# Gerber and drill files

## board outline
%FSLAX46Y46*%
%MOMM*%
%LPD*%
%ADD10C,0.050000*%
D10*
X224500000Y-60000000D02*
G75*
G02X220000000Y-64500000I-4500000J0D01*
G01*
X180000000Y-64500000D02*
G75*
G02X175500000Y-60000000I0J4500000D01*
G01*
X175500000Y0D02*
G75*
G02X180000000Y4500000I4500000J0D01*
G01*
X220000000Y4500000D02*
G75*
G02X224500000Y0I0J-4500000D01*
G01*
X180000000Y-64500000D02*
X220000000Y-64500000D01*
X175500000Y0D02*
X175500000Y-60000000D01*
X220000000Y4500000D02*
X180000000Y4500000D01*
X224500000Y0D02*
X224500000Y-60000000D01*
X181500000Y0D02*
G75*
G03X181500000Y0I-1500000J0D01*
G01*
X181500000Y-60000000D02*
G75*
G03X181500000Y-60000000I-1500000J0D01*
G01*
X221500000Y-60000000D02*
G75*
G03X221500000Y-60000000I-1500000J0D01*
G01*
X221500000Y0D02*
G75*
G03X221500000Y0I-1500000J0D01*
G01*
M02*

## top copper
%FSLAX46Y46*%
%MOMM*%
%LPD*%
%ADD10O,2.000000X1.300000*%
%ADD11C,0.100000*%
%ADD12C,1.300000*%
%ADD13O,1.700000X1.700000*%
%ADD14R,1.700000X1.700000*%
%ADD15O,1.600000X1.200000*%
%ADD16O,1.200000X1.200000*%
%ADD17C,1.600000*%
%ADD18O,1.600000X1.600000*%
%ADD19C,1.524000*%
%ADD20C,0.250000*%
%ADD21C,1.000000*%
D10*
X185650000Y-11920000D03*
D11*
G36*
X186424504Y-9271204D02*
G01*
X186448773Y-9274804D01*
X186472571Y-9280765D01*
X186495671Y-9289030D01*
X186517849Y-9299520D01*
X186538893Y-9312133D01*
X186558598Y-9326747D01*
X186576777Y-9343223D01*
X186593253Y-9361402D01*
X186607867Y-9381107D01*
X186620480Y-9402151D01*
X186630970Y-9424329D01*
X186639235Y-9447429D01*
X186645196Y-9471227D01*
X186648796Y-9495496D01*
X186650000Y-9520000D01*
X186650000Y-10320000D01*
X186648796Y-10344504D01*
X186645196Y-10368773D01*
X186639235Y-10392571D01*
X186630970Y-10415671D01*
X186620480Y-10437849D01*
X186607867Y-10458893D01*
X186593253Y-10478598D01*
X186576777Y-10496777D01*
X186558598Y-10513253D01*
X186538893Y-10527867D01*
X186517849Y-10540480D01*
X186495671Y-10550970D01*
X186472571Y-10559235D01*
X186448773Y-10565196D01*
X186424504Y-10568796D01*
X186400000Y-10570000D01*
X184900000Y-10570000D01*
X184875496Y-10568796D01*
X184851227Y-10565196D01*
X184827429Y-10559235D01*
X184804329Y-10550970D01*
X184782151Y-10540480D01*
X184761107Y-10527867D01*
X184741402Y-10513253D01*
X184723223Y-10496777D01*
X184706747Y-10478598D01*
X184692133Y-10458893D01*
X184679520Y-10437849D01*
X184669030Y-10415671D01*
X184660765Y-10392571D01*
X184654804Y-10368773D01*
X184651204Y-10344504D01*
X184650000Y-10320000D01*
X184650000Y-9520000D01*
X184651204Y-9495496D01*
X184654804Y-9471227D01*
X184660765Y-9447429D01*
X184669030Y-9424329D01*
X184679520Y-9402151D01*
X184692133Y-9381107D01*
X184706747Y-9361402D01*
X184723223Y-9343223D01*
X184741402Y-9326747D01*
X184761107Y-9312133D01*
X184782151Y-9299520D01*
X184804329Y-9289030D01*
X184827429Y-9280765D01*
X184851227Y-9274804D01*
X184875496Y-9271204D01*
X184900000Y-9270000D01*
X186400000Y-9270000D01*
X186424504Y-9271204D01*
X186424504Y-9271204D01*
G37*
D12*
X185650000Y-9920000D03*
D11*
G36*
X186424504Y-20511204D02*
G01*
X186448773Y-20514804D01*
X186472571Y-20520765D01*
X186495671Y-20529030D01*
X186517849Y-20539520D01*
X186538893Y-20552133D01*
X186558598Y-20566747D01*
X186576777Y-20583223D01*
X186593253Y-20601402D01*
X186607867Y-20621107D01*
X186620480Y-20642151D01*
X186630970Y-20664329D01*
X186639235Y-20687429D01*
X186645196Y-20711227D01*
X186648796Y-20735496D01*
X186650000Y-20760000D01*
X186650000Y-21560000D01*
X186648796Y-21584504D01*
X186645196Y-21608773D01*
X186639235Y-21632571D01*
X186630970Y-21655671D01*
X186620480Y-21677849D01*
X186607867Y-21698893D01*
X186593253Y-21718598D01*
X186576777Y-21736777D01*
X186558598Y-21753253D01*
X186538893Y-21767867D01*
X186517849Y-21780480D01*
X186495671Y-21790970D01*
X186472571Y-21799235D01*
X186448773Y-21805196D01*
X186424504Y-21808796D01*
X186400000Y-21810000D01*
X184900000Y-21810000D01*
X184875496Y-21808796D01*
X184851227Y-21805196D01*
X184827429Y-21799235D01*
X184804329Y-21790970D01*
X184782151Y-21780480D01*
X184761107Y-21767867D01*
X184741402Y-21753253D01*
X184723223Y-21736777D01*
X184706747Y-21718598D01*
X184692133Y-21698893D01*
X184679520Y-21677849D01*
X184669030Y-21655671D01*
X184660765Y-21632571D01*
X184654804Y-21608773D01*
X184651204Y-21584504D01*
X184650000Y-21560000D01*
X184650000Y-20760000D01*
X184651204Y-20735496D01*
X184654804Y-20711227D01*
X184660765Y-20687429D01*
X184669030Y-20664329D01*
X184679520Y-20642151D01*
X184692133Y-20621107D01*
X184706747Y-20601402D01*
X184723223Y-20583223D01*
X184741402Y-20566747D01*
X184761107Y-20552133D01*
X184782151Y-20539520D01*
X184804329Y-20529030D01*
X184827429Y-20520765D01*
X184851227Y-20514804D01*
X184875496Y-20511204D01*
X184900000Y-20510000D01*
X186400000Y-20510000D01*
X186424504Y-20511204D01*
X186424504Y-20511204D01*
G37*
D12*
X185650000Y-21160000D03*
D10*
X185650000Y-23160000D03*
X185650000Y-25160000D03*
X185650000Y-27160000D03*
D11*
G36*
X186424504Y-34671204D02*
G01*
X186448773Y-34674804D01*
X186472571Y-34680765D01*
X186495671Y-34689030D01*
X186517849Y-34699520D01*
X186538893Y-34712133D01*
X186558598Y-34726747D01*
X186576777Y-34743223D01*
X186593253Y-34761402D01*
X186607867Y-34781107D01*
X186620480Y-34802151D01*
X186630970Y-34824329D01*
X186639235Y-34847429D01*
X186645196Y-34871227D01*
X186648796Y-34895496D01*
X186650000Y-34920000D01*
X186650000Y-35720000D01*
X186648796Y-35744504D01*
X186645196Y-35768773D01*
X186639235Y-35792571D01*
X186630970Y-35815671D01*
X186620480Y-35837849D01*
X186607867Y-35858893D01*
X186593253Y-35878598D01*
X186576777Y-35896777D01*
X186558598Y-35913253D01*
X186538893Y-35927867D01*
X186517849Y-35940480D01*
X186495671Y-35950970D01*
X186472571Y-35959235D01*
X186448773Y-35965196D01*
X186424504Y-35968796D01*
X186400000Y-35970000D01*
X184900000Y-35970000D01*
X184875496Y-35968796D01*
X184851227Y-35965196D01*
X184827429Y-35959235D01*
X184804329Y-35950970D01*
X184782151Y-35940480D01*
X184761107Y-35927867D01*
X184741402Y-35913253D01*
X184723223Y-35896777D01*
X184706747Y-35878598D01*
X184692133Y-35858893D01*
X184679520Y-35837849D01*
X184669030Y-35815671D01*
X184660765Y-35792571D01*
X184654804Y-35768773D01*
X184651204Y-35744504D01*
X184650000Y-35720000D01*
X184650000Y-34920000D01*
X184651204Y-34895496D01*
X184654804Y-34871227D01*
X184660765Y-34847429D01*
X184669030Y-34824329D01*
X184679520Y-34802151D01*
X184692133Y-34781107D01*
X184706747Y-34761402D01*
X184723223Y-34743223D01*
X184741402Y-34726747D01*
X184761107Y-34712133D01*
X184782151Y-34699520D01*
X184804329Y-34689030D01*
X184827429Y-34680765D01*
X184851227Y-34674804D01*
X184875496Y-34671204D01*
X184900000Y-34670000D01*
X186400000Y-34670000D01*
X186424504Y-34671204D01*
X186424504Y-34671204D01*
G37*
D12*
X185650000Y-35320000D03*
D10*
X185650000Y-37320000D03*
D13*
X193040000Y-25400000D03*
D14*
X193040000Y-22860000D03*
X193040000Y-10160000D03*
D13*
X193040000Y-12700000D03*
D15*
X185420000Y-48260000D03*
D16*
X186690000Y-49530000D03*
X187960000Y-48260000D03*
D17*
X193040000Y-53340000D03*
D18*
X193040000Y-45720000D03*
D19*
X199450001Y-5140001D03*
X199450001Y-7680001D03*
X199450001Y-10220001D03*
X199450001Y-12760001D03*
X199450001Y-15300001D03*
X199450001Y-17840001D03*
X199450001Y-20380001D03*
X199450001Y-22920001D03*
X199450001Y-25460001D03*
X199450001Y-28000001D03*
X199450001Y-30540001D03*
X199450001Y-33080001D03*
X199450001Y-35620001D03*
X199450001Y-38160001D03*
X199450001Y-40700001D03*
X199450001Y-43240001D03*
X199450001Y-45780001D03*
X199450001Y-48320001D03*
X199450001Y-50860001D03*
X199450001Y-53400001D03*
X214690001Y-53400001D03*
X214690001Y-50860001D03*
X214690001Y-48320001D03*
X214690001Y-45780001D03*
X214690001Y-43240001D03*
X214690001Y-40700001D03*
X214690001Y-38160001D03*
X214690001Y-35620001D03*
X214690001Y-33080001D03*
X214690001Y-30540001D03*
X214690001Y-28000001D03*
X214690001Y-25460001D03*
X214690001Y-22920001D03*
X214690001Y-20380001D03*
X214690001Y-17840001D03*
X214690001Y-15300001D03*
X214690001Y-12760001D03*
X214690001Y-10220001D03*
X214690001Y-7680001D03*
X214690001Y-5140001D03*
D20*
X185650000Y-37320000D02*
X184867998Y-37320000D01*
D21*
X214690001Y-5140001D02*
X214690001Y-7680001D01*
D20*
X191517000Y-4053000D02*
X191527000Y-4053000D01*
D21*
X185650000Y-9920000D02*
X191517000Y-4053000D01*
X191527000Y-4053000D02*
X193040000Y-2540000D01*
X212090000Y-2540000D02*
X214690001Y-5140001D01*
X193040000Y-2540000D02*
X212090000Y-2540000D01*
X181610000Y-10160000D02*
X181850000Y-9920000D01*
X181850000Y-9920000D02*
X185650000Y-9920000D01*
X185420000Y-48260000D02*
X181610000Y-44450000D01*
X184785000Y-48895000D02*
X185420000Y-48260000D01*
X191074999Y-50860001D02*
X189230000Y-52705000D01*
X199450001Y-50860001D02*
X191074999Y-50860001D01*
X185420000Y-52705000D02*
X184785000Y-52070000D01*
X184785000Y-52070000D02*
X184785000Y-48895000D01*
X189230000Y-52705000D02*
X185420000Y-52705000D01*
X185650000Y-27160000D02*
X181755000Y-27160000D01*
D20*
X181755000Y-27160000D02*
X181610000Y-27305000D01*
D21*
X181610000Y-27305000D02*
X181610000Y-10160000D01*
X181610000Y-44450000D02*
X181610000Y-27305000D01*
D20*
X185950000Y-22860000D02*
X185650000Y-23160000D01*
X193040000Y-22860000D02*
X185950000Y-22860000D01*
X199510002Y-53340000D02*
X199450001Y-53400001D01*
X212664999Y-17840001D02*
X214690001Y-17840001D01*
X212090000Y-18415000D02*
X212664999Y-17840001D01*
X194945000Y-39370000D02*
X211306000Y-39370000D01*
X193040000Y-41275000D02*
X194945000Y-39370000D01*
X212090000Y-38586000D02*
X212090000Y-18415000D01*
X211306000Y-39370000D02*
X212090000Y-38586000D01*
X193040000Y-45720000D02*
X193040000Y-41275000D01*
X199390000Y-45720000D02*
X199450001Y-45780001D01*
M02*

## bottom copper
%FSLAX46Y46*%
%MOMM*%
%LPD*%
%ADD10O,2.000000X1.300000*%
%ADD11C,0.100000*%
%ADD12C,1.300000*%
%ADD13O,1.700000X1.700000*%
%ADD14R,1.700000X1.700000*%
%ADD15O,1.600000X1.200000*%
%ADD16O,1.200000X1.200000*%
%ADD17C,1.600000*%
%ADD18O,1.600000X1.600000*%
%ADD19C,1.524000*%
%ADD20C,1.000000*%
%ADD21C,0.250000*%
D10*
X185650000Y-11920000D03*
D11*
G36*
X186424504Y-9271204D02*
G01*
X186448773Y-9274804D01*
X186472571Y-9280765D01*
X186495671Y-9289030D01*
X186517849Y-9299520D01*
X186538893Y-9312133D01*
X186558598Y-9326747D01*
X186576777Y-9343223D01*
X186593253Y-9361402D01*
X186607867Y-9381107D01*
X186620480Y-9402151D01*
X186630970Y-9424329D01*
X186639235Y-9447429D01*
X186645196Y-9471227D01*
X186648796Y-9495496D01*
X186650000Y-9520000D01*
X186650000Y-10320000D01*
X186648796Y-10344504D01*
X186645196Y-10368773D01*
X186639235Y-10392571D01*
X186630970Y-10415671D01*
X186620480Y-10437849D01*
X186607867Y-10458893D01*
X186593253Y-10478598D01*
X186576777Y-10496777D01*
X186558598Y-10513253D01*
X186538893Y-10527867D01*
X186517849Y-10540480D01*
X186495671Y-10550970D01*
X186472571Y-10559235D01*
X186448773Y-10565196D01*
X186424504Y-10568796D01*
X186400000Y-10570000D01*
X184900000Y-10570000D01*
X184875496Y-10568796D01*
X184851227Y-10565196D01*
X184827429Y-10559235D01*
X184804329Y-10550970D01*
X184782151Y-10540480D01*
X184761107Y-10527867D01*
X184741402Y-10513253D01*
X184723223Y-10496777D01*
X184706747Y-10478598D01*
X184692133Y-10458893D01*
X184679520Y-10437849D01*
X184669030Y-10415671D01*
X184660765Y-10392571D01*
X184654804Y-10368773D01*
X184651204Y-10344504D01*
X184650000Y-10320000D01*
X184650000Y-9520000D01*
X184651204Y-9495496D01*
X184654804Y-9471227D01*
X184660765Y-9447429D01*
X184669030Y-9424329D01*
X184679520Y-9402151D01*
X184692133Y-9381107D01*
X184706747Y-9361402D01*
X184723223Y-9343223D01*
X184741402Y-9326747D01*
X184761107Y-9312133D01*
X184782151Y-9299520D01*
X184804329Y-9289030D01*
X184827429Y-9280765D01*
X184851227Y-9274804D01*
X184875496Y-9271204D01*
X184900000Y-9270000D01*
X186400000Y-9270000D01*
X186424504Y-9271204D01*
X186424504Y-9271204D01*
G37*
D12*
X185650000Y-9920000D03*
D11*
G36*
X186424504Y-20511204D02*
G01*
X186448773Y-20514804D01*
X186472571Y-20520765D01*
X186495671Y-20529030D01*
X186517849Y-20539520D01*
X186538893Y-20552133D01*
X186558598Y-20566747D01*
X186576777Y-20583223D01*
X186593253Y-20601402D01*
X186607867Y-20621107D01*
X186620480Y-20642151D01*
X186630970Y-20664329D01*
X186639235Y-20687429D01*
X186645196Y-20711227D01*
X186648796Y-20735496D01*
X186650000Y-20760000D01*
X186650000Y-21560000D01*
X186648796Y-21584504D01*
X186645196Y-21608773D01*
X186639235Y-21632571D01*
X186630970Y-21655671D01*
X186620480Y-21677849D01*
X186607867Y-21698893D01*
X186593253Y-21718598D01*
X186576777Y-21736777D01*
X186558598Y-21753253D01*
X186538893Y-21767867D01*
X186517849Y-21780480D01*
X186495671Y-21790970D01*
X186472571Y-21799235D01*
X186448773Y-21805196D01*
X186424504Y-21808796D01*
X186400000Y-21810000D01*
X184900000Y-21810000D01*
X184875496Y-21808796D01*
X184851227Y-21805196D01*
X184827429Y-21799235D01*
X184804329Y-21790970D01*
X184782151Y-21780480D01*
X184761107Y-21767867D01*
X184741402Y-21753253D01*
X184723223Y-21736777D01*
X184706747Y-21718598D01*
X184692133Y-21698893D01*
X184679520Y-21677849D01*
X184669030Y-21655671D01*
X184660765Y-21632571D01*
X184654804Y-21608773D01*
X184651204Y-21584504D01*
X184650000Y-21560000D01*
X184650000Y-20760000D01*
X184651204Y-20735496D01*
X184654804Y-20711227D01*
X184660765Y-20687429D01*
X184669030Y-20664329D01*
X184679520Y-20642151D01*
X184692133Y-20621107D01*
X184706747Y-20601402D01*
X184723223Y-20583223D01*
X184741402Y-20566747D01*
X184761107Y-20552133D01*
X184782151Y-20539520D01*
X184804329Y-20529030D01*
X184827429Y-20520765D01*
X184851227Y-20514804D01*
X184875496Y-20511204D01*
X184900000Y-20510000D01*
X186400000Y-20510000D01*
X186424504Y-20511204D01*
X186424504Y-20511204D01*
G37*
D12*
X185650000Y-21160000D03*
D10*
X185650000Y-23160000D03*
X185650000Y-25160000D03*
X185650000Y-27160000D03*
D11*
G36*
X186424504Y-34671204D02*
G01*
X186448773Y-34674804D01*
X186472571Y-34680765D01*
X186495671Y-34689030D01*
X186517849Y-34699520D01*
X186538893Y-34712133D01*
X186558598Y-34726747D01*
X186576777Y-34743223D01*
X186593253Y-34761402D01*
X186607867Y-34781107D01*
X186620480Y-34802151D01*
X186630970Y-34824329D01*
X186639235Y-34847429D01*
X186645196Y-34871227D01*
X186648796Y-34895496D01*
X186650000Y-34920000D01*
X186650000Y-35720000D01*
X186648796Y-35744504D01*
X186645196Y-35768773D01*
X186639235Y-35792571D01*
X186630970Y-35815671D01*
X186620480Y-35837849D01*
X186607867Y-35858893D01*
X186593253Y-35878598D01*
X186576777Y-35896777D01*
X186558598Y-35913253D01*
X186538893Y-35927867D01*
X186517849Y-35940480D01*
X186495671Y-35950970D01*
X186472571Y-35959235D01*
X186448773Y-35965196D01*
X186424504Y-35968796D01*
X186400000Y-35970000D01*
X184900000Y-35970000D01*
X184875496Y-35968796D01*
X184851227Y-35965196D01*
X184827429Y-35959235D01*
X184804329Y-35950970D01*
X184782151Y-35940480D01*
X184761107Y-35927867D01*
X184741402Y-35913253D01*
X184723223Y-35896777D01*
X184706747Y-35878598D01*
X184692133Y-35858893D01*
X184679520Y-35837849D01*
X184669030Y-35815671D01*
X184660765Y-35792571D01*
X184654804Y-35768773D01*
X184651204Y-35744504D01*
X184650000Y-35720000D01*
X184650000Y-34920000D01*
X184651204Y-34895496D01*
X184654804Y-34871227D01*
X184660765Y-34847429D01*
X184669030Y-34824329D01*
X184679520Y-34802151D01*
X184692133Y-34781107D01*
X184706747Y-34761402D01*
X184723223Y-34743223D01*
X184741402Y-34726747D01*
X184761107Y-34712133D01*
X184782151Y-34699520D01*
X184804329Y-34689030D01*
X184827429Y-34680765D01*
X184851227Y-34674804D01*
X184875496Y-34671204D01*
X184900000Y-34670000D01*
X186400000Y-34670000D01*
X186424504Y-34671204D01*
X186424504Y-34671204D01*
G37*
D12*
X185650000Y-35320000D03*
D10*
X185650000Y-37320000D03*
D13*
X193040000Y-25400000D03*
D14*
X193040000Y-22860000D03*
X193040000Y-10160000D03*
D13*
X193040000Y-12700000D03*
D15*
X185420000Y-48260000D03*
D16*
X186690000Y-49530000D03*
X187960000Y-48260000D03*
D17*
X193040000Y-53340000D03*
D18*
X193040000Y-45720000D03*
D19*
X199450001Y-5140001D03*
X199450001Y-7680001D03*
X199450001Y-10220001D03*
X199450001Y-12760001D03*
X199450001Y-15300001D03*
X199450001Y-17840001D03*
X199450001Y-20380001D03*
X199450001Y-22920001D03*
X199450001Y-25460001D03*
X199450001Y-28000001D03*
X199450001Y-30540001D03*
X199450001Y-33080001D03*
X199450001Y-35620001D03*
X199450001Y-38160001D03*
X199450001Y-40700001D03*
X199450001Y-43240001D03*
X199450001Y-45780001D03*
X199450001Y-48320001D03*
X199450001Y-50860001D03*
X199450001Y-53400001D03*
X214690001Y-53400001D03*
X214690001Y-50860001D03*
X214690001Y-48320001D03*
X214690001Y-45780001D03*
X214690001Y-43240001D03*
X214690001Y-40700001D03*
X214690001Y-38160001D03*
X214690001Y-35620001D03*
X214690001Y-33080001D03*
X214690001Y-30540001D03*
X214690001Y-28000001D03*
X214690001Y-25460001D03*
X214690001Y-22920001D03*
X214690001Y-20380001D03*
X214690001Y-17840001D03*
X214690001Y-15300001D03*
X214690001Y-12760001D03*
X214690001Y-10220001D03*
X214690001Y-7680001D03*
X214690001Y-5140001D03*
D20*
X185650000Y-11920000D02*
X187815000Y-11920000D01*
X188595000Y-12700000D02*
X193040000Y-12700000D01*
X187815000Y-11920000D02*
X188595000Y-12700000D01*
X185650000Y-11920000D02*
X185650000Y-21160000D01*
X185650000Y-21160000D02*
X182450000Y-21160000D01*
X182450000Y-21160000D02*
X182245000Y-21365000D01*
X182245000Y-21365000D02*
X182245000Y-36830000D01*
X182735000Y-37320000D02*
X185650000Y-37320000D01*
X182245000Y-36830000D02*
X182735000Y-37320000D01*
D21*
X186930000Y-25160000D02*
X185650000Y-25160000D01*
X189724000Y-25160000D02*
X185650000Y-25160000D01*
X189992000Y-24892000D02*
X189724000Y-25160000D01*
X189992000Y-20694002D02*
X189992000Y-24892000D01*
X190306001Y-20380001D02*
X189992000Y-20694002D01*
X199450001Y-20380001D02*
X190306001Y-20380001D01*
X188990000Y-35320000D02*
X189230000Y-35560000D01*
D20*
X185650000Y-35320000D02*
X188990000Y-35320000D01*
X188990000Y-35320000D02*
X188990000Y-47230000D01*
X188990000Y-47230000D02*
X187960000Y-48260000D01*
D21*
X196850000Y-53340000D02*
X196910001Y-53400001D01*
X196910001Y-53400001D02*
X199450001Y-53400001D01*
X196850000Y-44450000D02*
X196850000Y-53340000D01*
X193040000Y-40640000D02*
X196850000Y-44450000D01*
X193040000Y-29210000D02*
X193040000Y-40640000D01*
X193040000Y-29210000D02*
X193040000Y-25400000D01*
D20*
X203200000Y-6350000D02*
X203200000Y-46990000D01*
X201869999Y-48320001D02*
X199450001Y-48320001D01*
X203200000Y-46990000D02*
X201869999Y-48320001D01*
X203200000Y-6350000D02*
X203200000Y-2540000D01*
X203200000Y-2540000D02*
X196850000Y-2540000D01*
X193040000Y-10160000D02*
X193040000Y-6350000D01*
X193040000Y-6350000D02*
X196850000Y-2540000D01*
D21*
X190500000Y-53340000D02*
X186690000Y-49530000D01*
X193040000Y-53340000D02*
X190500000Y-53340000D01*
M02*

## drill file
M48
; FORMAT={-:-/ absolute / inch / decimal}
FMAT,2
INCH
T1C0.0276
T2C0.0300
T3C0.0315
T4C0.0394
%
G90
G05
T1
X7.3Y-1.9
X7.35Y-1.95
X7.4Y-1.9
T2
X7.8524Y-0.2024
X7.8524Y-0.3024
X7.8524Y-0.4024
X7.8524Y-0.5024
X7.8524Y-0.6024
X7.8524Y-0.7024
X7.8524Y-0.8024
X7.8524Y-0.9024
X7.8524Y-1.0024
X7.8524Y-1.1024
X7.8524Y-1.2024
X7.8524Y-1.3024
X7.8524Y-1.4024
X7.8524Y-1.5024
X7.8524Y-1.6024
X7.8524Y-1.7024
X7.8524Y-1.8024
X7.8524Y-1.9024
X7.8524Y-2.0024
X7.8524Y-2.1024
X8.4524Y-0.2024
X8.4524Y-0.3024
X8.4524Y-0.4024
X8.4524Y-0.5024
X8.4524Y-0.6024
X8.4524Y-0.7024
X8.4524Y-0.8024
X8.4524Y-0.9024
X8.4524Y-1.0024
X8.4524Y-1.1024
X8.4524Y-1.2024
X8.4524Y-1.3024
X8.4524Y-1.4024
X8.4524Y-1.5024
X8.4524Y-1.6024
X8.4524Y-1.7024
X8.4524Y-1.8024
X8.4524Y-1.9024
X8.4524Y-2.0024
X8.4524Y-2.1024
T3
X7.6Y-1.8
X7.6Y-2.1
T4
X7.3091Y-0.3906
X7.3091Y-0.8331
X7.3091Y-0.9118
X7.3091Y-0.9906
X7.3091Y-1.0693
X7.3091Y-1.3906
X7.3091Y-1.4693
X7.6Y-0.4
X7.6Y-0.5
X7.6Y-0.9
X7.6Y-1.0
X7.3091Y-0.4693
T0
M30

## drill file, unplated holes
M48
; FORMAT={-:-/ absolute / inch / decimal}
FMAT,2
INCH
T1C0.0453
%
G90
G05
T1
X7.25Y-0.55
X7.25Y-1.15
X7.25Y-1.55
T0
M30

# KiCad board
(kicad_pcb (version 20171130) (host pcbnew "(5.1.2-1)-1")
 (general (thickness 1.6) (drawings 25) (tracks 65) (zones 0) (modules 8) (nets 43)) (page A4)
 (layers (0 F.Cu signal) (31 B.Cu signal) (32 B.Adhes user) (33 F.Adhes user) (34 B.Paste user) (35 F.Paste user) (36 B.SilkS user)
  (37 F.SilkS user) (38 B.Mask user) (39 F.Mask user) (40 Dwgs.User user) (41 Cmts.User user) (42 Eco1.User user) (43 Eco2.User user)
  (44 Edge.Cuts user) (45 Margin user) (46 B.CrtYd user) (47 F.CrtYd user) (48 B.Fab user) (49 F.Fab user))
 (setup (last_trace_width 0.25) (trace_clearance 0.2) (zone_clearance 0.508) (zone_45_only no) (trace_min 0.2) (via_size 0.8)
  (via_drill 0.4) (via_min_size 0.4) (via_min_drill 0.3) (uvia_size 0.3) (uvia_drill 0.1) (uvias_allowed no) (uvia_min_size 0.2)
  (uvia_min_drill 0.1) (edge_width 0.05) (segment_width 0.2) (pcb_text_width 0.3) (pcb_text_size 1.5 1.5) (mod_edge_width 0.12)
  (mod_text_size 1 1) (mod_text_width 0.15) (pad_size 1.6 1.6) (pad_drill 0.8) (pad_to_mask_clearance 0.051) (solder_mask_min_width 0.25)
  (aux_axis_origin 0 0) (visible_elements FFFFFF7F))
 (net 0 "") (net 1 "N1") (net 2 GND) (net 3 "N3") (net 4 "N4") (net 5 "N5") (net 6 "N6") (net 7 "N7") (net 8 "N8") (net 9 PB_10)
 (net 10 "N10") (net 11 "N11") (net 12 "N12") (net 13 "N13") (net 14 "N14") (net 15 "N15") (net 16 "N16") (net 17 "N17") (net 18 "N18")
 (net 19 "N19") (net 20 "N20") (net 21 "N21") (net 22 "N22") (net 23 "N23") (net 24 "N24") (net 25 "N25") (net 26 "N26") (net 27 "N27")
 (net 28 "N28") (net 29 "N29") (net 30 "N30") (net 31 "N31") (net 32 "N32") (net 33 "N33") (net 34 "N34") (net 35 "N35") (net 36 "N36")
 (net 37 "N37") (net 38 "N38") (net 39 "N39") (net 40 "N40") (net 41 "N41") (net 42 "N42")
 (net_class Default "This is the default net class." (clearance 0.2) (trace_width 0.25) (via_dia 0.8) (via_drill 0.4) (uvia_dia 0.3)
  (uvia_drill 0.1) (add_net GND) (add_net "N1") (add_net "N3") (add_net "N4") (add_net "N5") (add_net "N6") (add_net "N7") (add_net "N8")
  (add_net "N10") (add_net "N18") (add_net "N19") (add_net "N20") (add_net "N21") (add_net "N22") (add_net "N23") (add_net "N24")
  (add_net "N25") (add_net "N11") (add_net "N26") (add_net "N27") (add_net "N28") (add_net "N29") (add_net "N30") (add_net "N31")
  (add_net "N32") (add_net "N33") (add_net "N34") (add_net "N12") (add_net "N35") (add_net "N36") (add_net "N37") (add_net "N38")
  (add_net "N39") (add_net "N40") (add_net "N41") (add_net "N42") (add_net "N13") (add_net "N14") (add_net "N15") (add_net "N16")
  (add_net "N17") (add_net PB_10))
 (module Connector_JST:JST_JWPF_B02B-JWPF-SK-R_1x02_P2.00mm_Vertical (layer F.Cu) (at 185.65 9.92)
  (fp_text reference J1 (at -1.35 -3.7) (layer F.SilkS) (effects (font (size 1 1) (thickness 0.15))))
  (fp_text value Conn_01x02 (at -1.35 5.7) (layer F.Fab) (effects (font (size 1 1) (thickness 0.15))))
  (pad "" np_thru_hole circle (at -1.5 4.05) (size 1.15 1.15) (drill 1.15) (layers *.Cu *.Mask))
  (pad 2 thru_hole oval (at 0 2) (size 2 1.3) (drill 1) (layers *.Cu *.Mask) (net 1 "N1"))
  (pad 1 thru_hole roundrect (at 0 0) (size 2 1.3) (drill 1) (layers *.Cu *.Mask) (roundrect_rratio 0.192308) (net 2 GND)))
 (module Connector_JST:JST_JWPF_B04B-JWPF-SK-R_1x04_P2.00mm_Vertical (layer F.Cu) (at 185.65 21.16)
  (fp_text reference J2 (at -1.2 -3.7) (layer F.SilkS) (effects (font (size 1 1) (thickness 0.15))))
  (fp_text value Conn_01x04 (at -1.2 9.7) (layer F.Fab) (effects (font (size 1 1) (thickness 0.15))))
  (pad 1 thru_hole roundrect (at 0 0) (size 2 1.3) (drill 1) (layers *.Cu *.Mask) (roundrect_rratio 0.192308) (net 1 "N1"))
  (pad 2 thru_hole oval (at 0 2) (size 2 1.3) (drill 1) (layers *.Cu *.Mask) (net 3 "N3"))
  (pad 3 thru_hole oval (at 0 4) (size 2 1.3) (drill 1) (layers *.Cu *.Mask) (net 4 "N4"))
  (pad 4 thru_hole oval (at 0 6) (size 2 1.3) (drill 1) (layers *.Cu *.Mask) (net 2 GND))
  (pad "" np_thru_hole circle (at -1.5 8.05) (size 1.15 1.15) (drill 1.15) (layers *.Cu *.Mask)))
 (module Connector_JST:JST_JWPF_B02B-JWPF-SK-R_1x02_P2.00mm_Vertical (layer F.Cu) (at 185.65 35.32)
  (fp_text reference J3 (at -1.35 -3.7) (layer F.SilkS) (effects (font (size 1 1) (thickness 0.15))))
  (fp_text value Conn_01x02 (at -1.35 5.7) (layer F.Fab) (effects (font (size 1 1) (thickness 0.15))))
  (pad 1 thru_hole roundrect (at 0 0) (size 2 1.3) (drill 1) (layers *.Cu *.Mask) (roundrect_rratio 0.192308) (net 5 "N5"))
  (pad 2 thru_hole oval (at 0 2) (size 2 1.3) (drill 1) (layers *.Cu *.Mask) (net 1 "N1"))
  (pad "" np_thru_hole circle (at -1.5 4.05) (size 1.15 1.15) (drill 1.15) (layers *.Cu *.Mask)))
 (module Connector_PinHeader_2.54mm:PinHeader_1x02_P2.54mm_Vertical (layer F.Cu) (at 193.04 22.86)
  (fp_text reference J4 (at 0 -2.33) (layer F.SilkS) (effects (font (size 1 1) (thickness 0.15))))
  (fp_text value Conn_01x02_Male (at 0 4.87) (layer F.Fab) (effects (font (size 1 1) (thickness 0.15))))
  (pad 2 thru_hole oval (at 0 2.54) (size 1.7 1.7) (drill 1) (layers *.Cu *.Mask) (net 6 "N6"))
  (pad 1 thru_hole rect (at 0 0) (size 1.7 1.7) (drill 1) (layers *.Cu *.Mask) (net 3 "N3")))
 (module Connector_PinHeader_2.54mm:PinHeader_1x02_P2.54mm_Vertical (layer F.Cu) (at 193.04 10.16)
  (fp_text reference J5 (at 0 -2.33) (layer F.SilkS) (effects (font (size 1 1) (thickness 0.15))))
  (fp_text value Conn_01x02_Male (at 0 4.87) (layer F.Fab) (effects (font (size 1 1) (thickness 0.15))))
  (pad 1 thru_hole rect (at 0 0) (size 1.7 1.7) (drill 1) (layers *.Cu *.Mask) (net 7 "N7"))
  (pad 2 thru_hole oval (at 0 2.54) (size 1.7 1.7) (drill 1) (layers *.Cu *.Mask) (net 1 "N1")))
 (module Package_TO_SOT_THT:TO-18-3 (layer F.Cu) (at 185.42 48.26)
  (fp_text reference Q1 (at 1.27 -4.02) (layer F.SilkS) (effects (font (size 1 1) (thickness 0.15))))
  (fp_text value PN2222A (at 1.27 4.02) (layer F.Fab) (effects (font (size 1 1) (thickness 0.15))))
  (pad 1 thru_hole oval (at 0 0) (size 1.6 1.2) (drill 0.7) (layers *.Cu *.Mask) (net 2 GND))
  (pad 2 thru_hole oval (at 1.27 1.27) (size 1.2 1.2) (drill 0.7) (layers *.Cu *.Mask) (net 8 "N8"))
  (pad 3 thru_hole oval (at 2.54 0) (size 1.2 1.2) (drill 0.7) (layers *.Cu *.Mask) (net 5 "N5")))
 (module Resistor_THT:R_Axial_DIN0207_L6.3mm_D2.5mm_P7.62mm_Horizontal (layer F.Cu) (at 193.04 53.34 90)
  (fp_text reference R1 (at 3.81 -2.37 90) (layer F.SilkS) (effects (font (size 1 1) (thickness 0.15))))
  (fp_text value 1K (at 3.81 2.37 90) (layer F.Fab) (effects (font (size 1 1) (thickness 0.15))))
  (pad 1 thru_hole circle (at 0 0 90) (size 1.6 1.6) (drill 0.8) (layers *.Cu *.Mask) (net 8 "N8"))
  (pad 2 thru_hole oval (at 7.62 0 90) (size 1.6 1.6) (drill 0.8) (layers *.Cu *.Mask) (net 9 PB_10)))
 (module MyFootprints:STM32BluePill (layer F.Cu) (at 199.450001 5.140001)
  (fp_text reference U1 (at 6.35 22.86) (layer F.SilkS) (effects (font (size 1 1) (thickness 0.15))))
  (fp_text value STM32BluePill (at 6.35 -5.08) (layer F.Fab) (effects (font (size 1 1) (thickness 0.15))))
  (pad 1 thru_hole circle (at 0 0) (size 1.524 1.524) (drill 0.762) (layers *.Cu *.Mask) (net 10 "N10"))
  (pad 2 thru_hole circle (at 0 2.54) (size 1.524 1.524) (drill 0.762) (layers *.Cu *.Mask) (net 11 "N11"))
  (pad 3 thru_hole circle (at 0 5.08) (size 1.524 1.524) (drill 0.762) (layers *.Cu *.Mask) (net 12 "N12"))
  (pad 4 thru_hole circle (at 0 7.62) (size 1.524 1.524) (drill 0.762) (layers *.Cu *.Mask) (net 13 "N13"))
  (pad 5 thru_hole circle (at 0 10.16) (size 1.524 1.524) (drill 0.762) (layers *.Cu *.Mask) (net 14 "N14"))
  (pad 6 thru_hole circle (at 0 12.7) (size 1.524 1.524) (drill 0.762) (layers *.Cu *.Mask) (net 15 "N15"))
  (pad 7 thru_hole circle (at 0 15.24) (size 1.524 1.524) (drill 0.762) (layers *.Cu *.Mask) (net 4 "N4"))
  (pad 8 thru_hole circle (at 0 17.78) (size 1.524 1.524) (drill 0.762) (layers *.Cu *.Mask) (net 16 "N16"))
  (pad 9 thru_hole circle (at 0 20.32) (size 1.524 1.524) (drill 0.762) (layers *.Cu *.Mask) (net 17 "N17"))
  (pad 10 thru_hole circle (at 0 22.86) (size 1.524 1.524) (drill 0.762) (layers *.Cu *.Mask) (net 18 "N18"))
  (pad 11 thru_hole circle (at 0 25.4) (size 1.524 1.524) (drill 0.762) (layers *.Cu *.Mask) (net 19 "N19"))
  (pad 12 thru_hole circle (at 0 27.94) (size 1.524 1.524) (drill 0.762) (layers *.Cu *.Mask) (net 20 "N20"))
  (pad 13 thru_hole circle (at 0 30.48) (size 1.524 1.524) (drill 0.762) (layers *.Cu *.Mask) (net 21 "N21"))
  (pad 14 thru_hole circle (at 0 33.02) (size 1.524 1.524) (drill 0.762) (layers *.Cu *.Mask) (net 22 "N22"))
  (pad 15 thru_hole circle (at 0 35.56) (size 1.524 1.524) (drill 0.762) (layers *.Cu *.Mask) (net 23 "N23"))
  (pad 16 thru_hole circle (at 0 38.1) (size 1.524 1.524) (drill 0.762) (layers *.Cu *.Mask) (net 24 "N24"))
  (pad 17 thru_hole circle (at 0 40.64) (size 1.524 1.524) (drill 0.762) (layers *.Cu *.Mask) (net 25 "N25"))
  (pad 18 thru_hole circle (at 0 43.18) (size 1.524 1.524) (drill 0.762) (layers *.Cu *.Mask) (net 7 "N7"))
  (pad 19 thru_hole circle (at 0 45.72) (size 1.524 1.524) (drill 0.762) (layers *.Cu *.Mask) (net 2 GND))
  (pad 20 thru_hole circle (at 0 48.26) (size 1.524 1.524) (drill 0.762) (layers *.Cu *.Mask) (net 6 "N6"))
  (pad 21 thru_hole circle (at 15.24 48.26) (size 1.524 1.524) (drill 0.762) (layers *.Cu *.Mask) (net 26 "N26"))
  (pad 22 thru_hole circle (at 15.24 45.72) (size 1.524 1.524) (drill 0.762) (layers *.Cu *.Mask) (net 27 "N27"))
  (pad 23 thru_hole circle (at 15.24 43.18) (size 1.524 1.524) (drill 0.762) (layers *.Cu *.Mask) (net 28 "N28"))
  (pad 24 thru_hole circle (at 15.24 40.64) (size 1.524 1.524) (drill 0.762) (layers *.Cu *.Mask) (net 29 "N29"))
  (pad 25 thru_hole circle (at 15.24 38.1) (size 1.524 1.524) (drill 0.762) (layers *.Cu *.Mask) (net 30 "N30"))
  (pad 26 thru_hole circle (at 15.24 35.56) (size 1.524 1.524) (drill 0.762) (layers *.Cu *.Mask) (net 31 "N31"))
  (pad 27 thru_hole circle (at 15.24 33.02) (size 1.524 1.524) (drill 0.762) (layers *.Cu *.Mask) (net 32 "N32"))
  (pad 28 thru_hole circle (at 15.24 30.48) (size 1.524 1.524) (drill 0.762) (layers *.Cu *.Mask) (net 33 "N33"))
  (pad 29 thru_hole circle (at 15.24 27.94) (size 1.524 1.524) (drill 0.762) (layers *.Cu *.Mask) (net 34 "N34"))
  (pad 30 thru_hole circle (at 15.24 25.4) (size 1.524 1.524) (drill 0.762) (layers *.Cu *.Mask) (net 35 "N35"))
  (pad 31 thru_hole circle (at 15.24 22.86) (size 1.524 1.524) (drill 0.762) (layers *.Cu *.Mask) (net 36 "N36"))
  (pad 32 thru_hole circle (at 15.24 20.32) (size 1.524 1.524) (drill 0.762) (layers *.Cu *.Mask) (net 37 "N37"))
  (pad 33 thru_hole circle (at 15.24 17.78) (size 1.524 1.524) (drill 0.762) (layers *.Cu *.Mask) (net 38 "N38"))
  (pad 34 thru_hole circle (at 15.24 15.24) (size 1.524 1.524) (drill 0.762) (layers *.Cu *.Mask) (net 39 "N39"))
  (pad 35 thru_hole circle (at 15.24 12.7) (size 1.524 1.524) (drill 0.762) (layers *.Cu *.Mask) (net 9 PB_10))
  (pad 36 thru_hole circle (at 15.24 10.16) (size 1.524 1.524) (drill 0.762) (layers *.Cu *.Mask) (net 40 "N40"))
  (pad 37 thru_hole circle (at 15.24 7.62) (size 1.524 1.524) (drill 0.762) (layers *.Cu *.Mask) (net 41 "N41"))
  (pad 38 thru_hole circle (at 15.24 5.08) (size 1.524 1.524) (drill 0.762) (layers *.Cu *.Mask) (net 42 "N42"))
  (pad 39 thru_hole circle (at 15.24 2.54) (size 1.524 1.524) (drill 0.762) (layers *.Cu *.Mask) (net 2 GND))
  (pad 40 thru_hole circle (at 15.24 0) (size 1.524 1.524) (drill 0.762) (layers *.Cu *.Mask) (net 2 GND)))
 (gr_arc (start 220 60) (end 220 64.5) (angle -90) (layer Edge.Cuts) (width 0.05))
 (gr_arc (start 180 60) (end 175.5 60) (angle -90) (layer Edge.Cuts) (width 0.05))
 (gr_arc (start 180 0) (end 180 -4.5) (angle -90) (layer Edge.Cuts) (width 0.05))
 (gr_arc (start 220 0) (end 224.5 0) (angle -90) (layer Edge.Cuts) (width 0.05))
 (gr_line (start 180 64.5) (end 220 64.5) (layer Edge.Cuts) (width 0.05))
 (gr_line (start 175.5 0) (end 175.5 60) (layer Edge.Cuts) (width 0.05))
 (gr_line (start 220 -4.5) (end 180 -4.5) (layer Edge.Cuts) (width 0.05))
 (gr_line (start 224.5 0) (end 224.5 60) (layer Edge.Cuts) (width 0.05))
 (gr_circle (center 180 0) (end 181.5 0) (layer Edge.Cuts) (width 0.05))
 (gr_circle (center 180 60) (end 181.5 60) (layer Edge.Cuts) (width 0.05))
 (gr_circle (center 220 60) (end 221.5 60) (layer Edge.Cuts) (width 0.05))
 (gr_circle (center 220 0) (end 221.5 0) (layer Edge.Cuts) (width 0.05))
 (segment (start 185.65 37.32) (end 184.867998 37.32) (width 0.25) (layer F.Cu) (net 1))
 (segment (start 185.65 11.92) (end 187.815 11.92) (width 1) (layer B.Cu) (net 1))
 (segment (start 188.595 12.7) (end 193.04 12.7) (width 1) (layer B.Cu) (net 1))
 (segment (start 187.815 11.92) (end 188.595 12.7) (width 1) (layer B.Cu) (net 1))
 (segment (start 185.65 11.92) (end 185.65 21.16) (width 1) (layer B.Cu) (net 1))
 (segment (start 185.65 21.16) (end 182.45 21.16) (width 1) (layer B.Cu) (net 1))
 (segment (start 182.45 21.16) (end 182.245 21.365) (width 1) (layer B.Cu) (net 1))
 (segment (start 182.245 21.365) (end 182.245 36.83) (width 1) (layer B.Cu) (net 1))
 (segment (start 182.735 37.32) (end 185.65 37.32) (width 1) (layer B.Cu) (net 1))
 (segment (start 182.245 36.83) (end 182.735 37.32) (width 1) (layer B.Cu) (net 1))
 (segment (start 214.690001 5.140001) (end 214.690001 7.680001) (width 1) (layer F.Cu) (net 2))
 (segment (start 191.517 4.053) (end 191.527 4.053) (width 0.25) (layer F.Cu) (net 2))
 (segment (start 185.65 9.92) (end 191.517 4.053) (width 1) (layer F.Cu) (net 2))
 (segment (start 191.527 4.053) (end 193.04 2.54) (width 1) (layer F.Cu) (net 2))
 (segment (start 212.09 2.54) (end 214.690001 5.140001) (width 1) (layer F.Cu) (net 2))
 (segment (start 193.04 2.54) (end 212.09 2.54) (width 1) (layer F.Cu) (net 2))
 (segment (start 181.61 10.16) (end 181.85 9.92) (width 1) (layer F.Cu) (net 2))
 (segment (start 181.85 9.92) (end 185.65 9.92) (width 1) (layer F.Cu) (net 2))
 (segment (start 185.42 48.26) (end 181.61 44.45) (width 1) (layer F.Cu) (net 2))
 (segment (start 184.785 48.895) (end 185.42 48.26) (width 1) (layer F.Cu) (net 2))
 (segment (start 191.074999 50.860001) (end 189.23 52.705) (width 1) (layer F.Cu) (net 2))
 (segment (start 199.450001 50.860001) (end 191.074999 50.860001) (width 1) (layer F.Cu) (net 2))
 (segment (start 185.42 52.705) (end 184.785 52.07) (width 1) (layer F.Cu) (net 2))
 (segment (start 184.785 52.07) (end 184.785 48.895) (width 1) (layer F.Cu) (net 2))
 (segment (start 189.23 52.705) (end 185.42 52.705) (width 1) (layer F.Cu) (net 2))
 (segment (start 185.65 27.16) (end 181.755 27.16) (width 1) (layer F.Cu) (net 2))
 (segment (start 181.755 27.16) (end 181.61 27.305) (width 0.25) (layer F.Cu) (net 2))
 (segment (start 181.61 27.305) (end 181.61 10.16) (width 1) (layer F.Cu) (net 2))
 (segment (start 181.61 44.45) (end 181.61 27.305) (width 1) (layer F.Cu) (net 2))
 (segment (start 185.95 22.86) (end 185.65 23.16) (width 0.25) (layer F.Cu) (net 3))
 (segment (start 193.04 22.86) (end 185.95 22.86) (width 0.25) (layer F.Cu) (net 3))
 (segment (start 186.93 25.16) (end 185.65 25.16) (width 0.25) (layer B.Cu) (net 4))
 (segment (start 189.724 25.16) (end 185.65 25.16) (width 0.25) (layer B.Cu) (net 4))
 (segment (start 189.992 24.892) (end 189.724 25.16) (width 0.25) (layer B.Cu) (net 4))
 (segment (start 189.992 20.694002) (end 189.992 24.892) (width 0.25) (layer B.Cu) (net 4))
 (segment (start 190.306001 20.380001) (end 189.992 20.694002) (width 0.25) (layer B.Cu) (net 4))
 (segment (start 199.450001 20.380001) (end 190.306001 20.380001) (width 0.25) (layer B.Cu) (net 4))
 (segment (start 188.99 35.32) (end 189.23 35.56) (width 0.25) (layer B.Cu) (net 5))
 (segment (start 185.65 35.32) (end 188.99 35.32) (width 1) (layer B.Cu) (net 5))
 (segment (start 188.99 35.32) (end 188.99 47.23) (width 1) (layer B.Cu) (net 5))
 (segment (start 188.99 47.23) (end 187.96 48.26) (width 1) (layer B.Cu) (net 5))
 (segment (start 199.510002 53.34) (end 199.450001 53.400001) (width 0.25) (layer F.Cu) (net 6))
 (segment (start 196.85 53.34) (end 196.910001 53.400001) (width 0.25) (layer B.Cu) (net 6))
 (segment (start 196.910001 53.400001) (end 199.450001 53.400001) (width 0.25) (layer B.Cu) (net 6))
 (segment (start 196.85 44.45) (end 196.85 53.34) (width 0.25) (layer B.Cu) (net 6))
 (segment (start 193.04 40.64) (end 196.85 44.45) (width 0.25) (layer B.Cu) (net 6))
 (segment (start 193.04 29.21) (end 193.04 40.64) (width 0.25) (layer B.Cu) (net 6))
 (segment (start 193.04 29.21) (end 193.04 25.4) (width 0.25) (layer B.Cu) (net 6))
 (segment (start 203.2 6.35) (end 203.2 46.99) (width 1) (layer B.Cu) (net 7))
 (segment (start 201.869999 48.320001) (end 199.450001 48.320001) (width 1) (layer B.Cu) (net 7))
 (segment (start 203.2 46.99) (end 201.869999 48.320001) (width 1) (layer B.Cu) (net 7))
 (segment (start 203.2 6.35) (end 203.2 2.54) (width 1) (layer B.Cu) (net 7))
 (segment (start 203.2 2.54) (end 196.85 2.54) (width 1) (layer B.Cu) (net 7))
 (segment (start 193.04 10.16) (end 193.04 6.35) (width 1) (layer B.Cu) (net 7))
 (segment (start 193.04 6.35) (end 196.85 2.54) (width 1) (layer B.Cu) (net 7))
 (segment (start 190.5 53.34) (end 186.69 49.53) (width 0.25) (layer B.Cu) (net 8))
 (segment (start 193.04 53.34) (end 190.5 53.34) (width 0.25) (layer B.Cu) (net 8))
 (segment (start 212.664999 17.840001) (end 214.690001 17.840001) (width 0.25) (layer F.Cu) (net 9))
 (segment (start 212.09 18.415) (end 212.664999 17.840001) (width 0.25) (layer F.Cu) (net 9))
 (segment (start 194.945 39.37) (end 211.306 39.37) (width 0.25) (layer F.Cu) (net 9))
 (segment (start 193.04 41.275) (end 194.945 39.37) (width 0.25) (layer F.Cu) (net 9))
 (segment (start 212.09 38.586) (end 212.09 18.415) (width 0.25) (layer F.Cu) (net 9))
 (segment (start 211.306 39.37) (end 212.09 38.586) (width 0.25) (layer F.Cu) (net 9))
 (segment (start 193.04 45.72) (end 193.04 41.275) (width 0.25) (layer F.Cu) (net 9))
 (segment (start 199.39 45.72) (end 199.450001 45.780001) (width 0.25) (layer F.Cu) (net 25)))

